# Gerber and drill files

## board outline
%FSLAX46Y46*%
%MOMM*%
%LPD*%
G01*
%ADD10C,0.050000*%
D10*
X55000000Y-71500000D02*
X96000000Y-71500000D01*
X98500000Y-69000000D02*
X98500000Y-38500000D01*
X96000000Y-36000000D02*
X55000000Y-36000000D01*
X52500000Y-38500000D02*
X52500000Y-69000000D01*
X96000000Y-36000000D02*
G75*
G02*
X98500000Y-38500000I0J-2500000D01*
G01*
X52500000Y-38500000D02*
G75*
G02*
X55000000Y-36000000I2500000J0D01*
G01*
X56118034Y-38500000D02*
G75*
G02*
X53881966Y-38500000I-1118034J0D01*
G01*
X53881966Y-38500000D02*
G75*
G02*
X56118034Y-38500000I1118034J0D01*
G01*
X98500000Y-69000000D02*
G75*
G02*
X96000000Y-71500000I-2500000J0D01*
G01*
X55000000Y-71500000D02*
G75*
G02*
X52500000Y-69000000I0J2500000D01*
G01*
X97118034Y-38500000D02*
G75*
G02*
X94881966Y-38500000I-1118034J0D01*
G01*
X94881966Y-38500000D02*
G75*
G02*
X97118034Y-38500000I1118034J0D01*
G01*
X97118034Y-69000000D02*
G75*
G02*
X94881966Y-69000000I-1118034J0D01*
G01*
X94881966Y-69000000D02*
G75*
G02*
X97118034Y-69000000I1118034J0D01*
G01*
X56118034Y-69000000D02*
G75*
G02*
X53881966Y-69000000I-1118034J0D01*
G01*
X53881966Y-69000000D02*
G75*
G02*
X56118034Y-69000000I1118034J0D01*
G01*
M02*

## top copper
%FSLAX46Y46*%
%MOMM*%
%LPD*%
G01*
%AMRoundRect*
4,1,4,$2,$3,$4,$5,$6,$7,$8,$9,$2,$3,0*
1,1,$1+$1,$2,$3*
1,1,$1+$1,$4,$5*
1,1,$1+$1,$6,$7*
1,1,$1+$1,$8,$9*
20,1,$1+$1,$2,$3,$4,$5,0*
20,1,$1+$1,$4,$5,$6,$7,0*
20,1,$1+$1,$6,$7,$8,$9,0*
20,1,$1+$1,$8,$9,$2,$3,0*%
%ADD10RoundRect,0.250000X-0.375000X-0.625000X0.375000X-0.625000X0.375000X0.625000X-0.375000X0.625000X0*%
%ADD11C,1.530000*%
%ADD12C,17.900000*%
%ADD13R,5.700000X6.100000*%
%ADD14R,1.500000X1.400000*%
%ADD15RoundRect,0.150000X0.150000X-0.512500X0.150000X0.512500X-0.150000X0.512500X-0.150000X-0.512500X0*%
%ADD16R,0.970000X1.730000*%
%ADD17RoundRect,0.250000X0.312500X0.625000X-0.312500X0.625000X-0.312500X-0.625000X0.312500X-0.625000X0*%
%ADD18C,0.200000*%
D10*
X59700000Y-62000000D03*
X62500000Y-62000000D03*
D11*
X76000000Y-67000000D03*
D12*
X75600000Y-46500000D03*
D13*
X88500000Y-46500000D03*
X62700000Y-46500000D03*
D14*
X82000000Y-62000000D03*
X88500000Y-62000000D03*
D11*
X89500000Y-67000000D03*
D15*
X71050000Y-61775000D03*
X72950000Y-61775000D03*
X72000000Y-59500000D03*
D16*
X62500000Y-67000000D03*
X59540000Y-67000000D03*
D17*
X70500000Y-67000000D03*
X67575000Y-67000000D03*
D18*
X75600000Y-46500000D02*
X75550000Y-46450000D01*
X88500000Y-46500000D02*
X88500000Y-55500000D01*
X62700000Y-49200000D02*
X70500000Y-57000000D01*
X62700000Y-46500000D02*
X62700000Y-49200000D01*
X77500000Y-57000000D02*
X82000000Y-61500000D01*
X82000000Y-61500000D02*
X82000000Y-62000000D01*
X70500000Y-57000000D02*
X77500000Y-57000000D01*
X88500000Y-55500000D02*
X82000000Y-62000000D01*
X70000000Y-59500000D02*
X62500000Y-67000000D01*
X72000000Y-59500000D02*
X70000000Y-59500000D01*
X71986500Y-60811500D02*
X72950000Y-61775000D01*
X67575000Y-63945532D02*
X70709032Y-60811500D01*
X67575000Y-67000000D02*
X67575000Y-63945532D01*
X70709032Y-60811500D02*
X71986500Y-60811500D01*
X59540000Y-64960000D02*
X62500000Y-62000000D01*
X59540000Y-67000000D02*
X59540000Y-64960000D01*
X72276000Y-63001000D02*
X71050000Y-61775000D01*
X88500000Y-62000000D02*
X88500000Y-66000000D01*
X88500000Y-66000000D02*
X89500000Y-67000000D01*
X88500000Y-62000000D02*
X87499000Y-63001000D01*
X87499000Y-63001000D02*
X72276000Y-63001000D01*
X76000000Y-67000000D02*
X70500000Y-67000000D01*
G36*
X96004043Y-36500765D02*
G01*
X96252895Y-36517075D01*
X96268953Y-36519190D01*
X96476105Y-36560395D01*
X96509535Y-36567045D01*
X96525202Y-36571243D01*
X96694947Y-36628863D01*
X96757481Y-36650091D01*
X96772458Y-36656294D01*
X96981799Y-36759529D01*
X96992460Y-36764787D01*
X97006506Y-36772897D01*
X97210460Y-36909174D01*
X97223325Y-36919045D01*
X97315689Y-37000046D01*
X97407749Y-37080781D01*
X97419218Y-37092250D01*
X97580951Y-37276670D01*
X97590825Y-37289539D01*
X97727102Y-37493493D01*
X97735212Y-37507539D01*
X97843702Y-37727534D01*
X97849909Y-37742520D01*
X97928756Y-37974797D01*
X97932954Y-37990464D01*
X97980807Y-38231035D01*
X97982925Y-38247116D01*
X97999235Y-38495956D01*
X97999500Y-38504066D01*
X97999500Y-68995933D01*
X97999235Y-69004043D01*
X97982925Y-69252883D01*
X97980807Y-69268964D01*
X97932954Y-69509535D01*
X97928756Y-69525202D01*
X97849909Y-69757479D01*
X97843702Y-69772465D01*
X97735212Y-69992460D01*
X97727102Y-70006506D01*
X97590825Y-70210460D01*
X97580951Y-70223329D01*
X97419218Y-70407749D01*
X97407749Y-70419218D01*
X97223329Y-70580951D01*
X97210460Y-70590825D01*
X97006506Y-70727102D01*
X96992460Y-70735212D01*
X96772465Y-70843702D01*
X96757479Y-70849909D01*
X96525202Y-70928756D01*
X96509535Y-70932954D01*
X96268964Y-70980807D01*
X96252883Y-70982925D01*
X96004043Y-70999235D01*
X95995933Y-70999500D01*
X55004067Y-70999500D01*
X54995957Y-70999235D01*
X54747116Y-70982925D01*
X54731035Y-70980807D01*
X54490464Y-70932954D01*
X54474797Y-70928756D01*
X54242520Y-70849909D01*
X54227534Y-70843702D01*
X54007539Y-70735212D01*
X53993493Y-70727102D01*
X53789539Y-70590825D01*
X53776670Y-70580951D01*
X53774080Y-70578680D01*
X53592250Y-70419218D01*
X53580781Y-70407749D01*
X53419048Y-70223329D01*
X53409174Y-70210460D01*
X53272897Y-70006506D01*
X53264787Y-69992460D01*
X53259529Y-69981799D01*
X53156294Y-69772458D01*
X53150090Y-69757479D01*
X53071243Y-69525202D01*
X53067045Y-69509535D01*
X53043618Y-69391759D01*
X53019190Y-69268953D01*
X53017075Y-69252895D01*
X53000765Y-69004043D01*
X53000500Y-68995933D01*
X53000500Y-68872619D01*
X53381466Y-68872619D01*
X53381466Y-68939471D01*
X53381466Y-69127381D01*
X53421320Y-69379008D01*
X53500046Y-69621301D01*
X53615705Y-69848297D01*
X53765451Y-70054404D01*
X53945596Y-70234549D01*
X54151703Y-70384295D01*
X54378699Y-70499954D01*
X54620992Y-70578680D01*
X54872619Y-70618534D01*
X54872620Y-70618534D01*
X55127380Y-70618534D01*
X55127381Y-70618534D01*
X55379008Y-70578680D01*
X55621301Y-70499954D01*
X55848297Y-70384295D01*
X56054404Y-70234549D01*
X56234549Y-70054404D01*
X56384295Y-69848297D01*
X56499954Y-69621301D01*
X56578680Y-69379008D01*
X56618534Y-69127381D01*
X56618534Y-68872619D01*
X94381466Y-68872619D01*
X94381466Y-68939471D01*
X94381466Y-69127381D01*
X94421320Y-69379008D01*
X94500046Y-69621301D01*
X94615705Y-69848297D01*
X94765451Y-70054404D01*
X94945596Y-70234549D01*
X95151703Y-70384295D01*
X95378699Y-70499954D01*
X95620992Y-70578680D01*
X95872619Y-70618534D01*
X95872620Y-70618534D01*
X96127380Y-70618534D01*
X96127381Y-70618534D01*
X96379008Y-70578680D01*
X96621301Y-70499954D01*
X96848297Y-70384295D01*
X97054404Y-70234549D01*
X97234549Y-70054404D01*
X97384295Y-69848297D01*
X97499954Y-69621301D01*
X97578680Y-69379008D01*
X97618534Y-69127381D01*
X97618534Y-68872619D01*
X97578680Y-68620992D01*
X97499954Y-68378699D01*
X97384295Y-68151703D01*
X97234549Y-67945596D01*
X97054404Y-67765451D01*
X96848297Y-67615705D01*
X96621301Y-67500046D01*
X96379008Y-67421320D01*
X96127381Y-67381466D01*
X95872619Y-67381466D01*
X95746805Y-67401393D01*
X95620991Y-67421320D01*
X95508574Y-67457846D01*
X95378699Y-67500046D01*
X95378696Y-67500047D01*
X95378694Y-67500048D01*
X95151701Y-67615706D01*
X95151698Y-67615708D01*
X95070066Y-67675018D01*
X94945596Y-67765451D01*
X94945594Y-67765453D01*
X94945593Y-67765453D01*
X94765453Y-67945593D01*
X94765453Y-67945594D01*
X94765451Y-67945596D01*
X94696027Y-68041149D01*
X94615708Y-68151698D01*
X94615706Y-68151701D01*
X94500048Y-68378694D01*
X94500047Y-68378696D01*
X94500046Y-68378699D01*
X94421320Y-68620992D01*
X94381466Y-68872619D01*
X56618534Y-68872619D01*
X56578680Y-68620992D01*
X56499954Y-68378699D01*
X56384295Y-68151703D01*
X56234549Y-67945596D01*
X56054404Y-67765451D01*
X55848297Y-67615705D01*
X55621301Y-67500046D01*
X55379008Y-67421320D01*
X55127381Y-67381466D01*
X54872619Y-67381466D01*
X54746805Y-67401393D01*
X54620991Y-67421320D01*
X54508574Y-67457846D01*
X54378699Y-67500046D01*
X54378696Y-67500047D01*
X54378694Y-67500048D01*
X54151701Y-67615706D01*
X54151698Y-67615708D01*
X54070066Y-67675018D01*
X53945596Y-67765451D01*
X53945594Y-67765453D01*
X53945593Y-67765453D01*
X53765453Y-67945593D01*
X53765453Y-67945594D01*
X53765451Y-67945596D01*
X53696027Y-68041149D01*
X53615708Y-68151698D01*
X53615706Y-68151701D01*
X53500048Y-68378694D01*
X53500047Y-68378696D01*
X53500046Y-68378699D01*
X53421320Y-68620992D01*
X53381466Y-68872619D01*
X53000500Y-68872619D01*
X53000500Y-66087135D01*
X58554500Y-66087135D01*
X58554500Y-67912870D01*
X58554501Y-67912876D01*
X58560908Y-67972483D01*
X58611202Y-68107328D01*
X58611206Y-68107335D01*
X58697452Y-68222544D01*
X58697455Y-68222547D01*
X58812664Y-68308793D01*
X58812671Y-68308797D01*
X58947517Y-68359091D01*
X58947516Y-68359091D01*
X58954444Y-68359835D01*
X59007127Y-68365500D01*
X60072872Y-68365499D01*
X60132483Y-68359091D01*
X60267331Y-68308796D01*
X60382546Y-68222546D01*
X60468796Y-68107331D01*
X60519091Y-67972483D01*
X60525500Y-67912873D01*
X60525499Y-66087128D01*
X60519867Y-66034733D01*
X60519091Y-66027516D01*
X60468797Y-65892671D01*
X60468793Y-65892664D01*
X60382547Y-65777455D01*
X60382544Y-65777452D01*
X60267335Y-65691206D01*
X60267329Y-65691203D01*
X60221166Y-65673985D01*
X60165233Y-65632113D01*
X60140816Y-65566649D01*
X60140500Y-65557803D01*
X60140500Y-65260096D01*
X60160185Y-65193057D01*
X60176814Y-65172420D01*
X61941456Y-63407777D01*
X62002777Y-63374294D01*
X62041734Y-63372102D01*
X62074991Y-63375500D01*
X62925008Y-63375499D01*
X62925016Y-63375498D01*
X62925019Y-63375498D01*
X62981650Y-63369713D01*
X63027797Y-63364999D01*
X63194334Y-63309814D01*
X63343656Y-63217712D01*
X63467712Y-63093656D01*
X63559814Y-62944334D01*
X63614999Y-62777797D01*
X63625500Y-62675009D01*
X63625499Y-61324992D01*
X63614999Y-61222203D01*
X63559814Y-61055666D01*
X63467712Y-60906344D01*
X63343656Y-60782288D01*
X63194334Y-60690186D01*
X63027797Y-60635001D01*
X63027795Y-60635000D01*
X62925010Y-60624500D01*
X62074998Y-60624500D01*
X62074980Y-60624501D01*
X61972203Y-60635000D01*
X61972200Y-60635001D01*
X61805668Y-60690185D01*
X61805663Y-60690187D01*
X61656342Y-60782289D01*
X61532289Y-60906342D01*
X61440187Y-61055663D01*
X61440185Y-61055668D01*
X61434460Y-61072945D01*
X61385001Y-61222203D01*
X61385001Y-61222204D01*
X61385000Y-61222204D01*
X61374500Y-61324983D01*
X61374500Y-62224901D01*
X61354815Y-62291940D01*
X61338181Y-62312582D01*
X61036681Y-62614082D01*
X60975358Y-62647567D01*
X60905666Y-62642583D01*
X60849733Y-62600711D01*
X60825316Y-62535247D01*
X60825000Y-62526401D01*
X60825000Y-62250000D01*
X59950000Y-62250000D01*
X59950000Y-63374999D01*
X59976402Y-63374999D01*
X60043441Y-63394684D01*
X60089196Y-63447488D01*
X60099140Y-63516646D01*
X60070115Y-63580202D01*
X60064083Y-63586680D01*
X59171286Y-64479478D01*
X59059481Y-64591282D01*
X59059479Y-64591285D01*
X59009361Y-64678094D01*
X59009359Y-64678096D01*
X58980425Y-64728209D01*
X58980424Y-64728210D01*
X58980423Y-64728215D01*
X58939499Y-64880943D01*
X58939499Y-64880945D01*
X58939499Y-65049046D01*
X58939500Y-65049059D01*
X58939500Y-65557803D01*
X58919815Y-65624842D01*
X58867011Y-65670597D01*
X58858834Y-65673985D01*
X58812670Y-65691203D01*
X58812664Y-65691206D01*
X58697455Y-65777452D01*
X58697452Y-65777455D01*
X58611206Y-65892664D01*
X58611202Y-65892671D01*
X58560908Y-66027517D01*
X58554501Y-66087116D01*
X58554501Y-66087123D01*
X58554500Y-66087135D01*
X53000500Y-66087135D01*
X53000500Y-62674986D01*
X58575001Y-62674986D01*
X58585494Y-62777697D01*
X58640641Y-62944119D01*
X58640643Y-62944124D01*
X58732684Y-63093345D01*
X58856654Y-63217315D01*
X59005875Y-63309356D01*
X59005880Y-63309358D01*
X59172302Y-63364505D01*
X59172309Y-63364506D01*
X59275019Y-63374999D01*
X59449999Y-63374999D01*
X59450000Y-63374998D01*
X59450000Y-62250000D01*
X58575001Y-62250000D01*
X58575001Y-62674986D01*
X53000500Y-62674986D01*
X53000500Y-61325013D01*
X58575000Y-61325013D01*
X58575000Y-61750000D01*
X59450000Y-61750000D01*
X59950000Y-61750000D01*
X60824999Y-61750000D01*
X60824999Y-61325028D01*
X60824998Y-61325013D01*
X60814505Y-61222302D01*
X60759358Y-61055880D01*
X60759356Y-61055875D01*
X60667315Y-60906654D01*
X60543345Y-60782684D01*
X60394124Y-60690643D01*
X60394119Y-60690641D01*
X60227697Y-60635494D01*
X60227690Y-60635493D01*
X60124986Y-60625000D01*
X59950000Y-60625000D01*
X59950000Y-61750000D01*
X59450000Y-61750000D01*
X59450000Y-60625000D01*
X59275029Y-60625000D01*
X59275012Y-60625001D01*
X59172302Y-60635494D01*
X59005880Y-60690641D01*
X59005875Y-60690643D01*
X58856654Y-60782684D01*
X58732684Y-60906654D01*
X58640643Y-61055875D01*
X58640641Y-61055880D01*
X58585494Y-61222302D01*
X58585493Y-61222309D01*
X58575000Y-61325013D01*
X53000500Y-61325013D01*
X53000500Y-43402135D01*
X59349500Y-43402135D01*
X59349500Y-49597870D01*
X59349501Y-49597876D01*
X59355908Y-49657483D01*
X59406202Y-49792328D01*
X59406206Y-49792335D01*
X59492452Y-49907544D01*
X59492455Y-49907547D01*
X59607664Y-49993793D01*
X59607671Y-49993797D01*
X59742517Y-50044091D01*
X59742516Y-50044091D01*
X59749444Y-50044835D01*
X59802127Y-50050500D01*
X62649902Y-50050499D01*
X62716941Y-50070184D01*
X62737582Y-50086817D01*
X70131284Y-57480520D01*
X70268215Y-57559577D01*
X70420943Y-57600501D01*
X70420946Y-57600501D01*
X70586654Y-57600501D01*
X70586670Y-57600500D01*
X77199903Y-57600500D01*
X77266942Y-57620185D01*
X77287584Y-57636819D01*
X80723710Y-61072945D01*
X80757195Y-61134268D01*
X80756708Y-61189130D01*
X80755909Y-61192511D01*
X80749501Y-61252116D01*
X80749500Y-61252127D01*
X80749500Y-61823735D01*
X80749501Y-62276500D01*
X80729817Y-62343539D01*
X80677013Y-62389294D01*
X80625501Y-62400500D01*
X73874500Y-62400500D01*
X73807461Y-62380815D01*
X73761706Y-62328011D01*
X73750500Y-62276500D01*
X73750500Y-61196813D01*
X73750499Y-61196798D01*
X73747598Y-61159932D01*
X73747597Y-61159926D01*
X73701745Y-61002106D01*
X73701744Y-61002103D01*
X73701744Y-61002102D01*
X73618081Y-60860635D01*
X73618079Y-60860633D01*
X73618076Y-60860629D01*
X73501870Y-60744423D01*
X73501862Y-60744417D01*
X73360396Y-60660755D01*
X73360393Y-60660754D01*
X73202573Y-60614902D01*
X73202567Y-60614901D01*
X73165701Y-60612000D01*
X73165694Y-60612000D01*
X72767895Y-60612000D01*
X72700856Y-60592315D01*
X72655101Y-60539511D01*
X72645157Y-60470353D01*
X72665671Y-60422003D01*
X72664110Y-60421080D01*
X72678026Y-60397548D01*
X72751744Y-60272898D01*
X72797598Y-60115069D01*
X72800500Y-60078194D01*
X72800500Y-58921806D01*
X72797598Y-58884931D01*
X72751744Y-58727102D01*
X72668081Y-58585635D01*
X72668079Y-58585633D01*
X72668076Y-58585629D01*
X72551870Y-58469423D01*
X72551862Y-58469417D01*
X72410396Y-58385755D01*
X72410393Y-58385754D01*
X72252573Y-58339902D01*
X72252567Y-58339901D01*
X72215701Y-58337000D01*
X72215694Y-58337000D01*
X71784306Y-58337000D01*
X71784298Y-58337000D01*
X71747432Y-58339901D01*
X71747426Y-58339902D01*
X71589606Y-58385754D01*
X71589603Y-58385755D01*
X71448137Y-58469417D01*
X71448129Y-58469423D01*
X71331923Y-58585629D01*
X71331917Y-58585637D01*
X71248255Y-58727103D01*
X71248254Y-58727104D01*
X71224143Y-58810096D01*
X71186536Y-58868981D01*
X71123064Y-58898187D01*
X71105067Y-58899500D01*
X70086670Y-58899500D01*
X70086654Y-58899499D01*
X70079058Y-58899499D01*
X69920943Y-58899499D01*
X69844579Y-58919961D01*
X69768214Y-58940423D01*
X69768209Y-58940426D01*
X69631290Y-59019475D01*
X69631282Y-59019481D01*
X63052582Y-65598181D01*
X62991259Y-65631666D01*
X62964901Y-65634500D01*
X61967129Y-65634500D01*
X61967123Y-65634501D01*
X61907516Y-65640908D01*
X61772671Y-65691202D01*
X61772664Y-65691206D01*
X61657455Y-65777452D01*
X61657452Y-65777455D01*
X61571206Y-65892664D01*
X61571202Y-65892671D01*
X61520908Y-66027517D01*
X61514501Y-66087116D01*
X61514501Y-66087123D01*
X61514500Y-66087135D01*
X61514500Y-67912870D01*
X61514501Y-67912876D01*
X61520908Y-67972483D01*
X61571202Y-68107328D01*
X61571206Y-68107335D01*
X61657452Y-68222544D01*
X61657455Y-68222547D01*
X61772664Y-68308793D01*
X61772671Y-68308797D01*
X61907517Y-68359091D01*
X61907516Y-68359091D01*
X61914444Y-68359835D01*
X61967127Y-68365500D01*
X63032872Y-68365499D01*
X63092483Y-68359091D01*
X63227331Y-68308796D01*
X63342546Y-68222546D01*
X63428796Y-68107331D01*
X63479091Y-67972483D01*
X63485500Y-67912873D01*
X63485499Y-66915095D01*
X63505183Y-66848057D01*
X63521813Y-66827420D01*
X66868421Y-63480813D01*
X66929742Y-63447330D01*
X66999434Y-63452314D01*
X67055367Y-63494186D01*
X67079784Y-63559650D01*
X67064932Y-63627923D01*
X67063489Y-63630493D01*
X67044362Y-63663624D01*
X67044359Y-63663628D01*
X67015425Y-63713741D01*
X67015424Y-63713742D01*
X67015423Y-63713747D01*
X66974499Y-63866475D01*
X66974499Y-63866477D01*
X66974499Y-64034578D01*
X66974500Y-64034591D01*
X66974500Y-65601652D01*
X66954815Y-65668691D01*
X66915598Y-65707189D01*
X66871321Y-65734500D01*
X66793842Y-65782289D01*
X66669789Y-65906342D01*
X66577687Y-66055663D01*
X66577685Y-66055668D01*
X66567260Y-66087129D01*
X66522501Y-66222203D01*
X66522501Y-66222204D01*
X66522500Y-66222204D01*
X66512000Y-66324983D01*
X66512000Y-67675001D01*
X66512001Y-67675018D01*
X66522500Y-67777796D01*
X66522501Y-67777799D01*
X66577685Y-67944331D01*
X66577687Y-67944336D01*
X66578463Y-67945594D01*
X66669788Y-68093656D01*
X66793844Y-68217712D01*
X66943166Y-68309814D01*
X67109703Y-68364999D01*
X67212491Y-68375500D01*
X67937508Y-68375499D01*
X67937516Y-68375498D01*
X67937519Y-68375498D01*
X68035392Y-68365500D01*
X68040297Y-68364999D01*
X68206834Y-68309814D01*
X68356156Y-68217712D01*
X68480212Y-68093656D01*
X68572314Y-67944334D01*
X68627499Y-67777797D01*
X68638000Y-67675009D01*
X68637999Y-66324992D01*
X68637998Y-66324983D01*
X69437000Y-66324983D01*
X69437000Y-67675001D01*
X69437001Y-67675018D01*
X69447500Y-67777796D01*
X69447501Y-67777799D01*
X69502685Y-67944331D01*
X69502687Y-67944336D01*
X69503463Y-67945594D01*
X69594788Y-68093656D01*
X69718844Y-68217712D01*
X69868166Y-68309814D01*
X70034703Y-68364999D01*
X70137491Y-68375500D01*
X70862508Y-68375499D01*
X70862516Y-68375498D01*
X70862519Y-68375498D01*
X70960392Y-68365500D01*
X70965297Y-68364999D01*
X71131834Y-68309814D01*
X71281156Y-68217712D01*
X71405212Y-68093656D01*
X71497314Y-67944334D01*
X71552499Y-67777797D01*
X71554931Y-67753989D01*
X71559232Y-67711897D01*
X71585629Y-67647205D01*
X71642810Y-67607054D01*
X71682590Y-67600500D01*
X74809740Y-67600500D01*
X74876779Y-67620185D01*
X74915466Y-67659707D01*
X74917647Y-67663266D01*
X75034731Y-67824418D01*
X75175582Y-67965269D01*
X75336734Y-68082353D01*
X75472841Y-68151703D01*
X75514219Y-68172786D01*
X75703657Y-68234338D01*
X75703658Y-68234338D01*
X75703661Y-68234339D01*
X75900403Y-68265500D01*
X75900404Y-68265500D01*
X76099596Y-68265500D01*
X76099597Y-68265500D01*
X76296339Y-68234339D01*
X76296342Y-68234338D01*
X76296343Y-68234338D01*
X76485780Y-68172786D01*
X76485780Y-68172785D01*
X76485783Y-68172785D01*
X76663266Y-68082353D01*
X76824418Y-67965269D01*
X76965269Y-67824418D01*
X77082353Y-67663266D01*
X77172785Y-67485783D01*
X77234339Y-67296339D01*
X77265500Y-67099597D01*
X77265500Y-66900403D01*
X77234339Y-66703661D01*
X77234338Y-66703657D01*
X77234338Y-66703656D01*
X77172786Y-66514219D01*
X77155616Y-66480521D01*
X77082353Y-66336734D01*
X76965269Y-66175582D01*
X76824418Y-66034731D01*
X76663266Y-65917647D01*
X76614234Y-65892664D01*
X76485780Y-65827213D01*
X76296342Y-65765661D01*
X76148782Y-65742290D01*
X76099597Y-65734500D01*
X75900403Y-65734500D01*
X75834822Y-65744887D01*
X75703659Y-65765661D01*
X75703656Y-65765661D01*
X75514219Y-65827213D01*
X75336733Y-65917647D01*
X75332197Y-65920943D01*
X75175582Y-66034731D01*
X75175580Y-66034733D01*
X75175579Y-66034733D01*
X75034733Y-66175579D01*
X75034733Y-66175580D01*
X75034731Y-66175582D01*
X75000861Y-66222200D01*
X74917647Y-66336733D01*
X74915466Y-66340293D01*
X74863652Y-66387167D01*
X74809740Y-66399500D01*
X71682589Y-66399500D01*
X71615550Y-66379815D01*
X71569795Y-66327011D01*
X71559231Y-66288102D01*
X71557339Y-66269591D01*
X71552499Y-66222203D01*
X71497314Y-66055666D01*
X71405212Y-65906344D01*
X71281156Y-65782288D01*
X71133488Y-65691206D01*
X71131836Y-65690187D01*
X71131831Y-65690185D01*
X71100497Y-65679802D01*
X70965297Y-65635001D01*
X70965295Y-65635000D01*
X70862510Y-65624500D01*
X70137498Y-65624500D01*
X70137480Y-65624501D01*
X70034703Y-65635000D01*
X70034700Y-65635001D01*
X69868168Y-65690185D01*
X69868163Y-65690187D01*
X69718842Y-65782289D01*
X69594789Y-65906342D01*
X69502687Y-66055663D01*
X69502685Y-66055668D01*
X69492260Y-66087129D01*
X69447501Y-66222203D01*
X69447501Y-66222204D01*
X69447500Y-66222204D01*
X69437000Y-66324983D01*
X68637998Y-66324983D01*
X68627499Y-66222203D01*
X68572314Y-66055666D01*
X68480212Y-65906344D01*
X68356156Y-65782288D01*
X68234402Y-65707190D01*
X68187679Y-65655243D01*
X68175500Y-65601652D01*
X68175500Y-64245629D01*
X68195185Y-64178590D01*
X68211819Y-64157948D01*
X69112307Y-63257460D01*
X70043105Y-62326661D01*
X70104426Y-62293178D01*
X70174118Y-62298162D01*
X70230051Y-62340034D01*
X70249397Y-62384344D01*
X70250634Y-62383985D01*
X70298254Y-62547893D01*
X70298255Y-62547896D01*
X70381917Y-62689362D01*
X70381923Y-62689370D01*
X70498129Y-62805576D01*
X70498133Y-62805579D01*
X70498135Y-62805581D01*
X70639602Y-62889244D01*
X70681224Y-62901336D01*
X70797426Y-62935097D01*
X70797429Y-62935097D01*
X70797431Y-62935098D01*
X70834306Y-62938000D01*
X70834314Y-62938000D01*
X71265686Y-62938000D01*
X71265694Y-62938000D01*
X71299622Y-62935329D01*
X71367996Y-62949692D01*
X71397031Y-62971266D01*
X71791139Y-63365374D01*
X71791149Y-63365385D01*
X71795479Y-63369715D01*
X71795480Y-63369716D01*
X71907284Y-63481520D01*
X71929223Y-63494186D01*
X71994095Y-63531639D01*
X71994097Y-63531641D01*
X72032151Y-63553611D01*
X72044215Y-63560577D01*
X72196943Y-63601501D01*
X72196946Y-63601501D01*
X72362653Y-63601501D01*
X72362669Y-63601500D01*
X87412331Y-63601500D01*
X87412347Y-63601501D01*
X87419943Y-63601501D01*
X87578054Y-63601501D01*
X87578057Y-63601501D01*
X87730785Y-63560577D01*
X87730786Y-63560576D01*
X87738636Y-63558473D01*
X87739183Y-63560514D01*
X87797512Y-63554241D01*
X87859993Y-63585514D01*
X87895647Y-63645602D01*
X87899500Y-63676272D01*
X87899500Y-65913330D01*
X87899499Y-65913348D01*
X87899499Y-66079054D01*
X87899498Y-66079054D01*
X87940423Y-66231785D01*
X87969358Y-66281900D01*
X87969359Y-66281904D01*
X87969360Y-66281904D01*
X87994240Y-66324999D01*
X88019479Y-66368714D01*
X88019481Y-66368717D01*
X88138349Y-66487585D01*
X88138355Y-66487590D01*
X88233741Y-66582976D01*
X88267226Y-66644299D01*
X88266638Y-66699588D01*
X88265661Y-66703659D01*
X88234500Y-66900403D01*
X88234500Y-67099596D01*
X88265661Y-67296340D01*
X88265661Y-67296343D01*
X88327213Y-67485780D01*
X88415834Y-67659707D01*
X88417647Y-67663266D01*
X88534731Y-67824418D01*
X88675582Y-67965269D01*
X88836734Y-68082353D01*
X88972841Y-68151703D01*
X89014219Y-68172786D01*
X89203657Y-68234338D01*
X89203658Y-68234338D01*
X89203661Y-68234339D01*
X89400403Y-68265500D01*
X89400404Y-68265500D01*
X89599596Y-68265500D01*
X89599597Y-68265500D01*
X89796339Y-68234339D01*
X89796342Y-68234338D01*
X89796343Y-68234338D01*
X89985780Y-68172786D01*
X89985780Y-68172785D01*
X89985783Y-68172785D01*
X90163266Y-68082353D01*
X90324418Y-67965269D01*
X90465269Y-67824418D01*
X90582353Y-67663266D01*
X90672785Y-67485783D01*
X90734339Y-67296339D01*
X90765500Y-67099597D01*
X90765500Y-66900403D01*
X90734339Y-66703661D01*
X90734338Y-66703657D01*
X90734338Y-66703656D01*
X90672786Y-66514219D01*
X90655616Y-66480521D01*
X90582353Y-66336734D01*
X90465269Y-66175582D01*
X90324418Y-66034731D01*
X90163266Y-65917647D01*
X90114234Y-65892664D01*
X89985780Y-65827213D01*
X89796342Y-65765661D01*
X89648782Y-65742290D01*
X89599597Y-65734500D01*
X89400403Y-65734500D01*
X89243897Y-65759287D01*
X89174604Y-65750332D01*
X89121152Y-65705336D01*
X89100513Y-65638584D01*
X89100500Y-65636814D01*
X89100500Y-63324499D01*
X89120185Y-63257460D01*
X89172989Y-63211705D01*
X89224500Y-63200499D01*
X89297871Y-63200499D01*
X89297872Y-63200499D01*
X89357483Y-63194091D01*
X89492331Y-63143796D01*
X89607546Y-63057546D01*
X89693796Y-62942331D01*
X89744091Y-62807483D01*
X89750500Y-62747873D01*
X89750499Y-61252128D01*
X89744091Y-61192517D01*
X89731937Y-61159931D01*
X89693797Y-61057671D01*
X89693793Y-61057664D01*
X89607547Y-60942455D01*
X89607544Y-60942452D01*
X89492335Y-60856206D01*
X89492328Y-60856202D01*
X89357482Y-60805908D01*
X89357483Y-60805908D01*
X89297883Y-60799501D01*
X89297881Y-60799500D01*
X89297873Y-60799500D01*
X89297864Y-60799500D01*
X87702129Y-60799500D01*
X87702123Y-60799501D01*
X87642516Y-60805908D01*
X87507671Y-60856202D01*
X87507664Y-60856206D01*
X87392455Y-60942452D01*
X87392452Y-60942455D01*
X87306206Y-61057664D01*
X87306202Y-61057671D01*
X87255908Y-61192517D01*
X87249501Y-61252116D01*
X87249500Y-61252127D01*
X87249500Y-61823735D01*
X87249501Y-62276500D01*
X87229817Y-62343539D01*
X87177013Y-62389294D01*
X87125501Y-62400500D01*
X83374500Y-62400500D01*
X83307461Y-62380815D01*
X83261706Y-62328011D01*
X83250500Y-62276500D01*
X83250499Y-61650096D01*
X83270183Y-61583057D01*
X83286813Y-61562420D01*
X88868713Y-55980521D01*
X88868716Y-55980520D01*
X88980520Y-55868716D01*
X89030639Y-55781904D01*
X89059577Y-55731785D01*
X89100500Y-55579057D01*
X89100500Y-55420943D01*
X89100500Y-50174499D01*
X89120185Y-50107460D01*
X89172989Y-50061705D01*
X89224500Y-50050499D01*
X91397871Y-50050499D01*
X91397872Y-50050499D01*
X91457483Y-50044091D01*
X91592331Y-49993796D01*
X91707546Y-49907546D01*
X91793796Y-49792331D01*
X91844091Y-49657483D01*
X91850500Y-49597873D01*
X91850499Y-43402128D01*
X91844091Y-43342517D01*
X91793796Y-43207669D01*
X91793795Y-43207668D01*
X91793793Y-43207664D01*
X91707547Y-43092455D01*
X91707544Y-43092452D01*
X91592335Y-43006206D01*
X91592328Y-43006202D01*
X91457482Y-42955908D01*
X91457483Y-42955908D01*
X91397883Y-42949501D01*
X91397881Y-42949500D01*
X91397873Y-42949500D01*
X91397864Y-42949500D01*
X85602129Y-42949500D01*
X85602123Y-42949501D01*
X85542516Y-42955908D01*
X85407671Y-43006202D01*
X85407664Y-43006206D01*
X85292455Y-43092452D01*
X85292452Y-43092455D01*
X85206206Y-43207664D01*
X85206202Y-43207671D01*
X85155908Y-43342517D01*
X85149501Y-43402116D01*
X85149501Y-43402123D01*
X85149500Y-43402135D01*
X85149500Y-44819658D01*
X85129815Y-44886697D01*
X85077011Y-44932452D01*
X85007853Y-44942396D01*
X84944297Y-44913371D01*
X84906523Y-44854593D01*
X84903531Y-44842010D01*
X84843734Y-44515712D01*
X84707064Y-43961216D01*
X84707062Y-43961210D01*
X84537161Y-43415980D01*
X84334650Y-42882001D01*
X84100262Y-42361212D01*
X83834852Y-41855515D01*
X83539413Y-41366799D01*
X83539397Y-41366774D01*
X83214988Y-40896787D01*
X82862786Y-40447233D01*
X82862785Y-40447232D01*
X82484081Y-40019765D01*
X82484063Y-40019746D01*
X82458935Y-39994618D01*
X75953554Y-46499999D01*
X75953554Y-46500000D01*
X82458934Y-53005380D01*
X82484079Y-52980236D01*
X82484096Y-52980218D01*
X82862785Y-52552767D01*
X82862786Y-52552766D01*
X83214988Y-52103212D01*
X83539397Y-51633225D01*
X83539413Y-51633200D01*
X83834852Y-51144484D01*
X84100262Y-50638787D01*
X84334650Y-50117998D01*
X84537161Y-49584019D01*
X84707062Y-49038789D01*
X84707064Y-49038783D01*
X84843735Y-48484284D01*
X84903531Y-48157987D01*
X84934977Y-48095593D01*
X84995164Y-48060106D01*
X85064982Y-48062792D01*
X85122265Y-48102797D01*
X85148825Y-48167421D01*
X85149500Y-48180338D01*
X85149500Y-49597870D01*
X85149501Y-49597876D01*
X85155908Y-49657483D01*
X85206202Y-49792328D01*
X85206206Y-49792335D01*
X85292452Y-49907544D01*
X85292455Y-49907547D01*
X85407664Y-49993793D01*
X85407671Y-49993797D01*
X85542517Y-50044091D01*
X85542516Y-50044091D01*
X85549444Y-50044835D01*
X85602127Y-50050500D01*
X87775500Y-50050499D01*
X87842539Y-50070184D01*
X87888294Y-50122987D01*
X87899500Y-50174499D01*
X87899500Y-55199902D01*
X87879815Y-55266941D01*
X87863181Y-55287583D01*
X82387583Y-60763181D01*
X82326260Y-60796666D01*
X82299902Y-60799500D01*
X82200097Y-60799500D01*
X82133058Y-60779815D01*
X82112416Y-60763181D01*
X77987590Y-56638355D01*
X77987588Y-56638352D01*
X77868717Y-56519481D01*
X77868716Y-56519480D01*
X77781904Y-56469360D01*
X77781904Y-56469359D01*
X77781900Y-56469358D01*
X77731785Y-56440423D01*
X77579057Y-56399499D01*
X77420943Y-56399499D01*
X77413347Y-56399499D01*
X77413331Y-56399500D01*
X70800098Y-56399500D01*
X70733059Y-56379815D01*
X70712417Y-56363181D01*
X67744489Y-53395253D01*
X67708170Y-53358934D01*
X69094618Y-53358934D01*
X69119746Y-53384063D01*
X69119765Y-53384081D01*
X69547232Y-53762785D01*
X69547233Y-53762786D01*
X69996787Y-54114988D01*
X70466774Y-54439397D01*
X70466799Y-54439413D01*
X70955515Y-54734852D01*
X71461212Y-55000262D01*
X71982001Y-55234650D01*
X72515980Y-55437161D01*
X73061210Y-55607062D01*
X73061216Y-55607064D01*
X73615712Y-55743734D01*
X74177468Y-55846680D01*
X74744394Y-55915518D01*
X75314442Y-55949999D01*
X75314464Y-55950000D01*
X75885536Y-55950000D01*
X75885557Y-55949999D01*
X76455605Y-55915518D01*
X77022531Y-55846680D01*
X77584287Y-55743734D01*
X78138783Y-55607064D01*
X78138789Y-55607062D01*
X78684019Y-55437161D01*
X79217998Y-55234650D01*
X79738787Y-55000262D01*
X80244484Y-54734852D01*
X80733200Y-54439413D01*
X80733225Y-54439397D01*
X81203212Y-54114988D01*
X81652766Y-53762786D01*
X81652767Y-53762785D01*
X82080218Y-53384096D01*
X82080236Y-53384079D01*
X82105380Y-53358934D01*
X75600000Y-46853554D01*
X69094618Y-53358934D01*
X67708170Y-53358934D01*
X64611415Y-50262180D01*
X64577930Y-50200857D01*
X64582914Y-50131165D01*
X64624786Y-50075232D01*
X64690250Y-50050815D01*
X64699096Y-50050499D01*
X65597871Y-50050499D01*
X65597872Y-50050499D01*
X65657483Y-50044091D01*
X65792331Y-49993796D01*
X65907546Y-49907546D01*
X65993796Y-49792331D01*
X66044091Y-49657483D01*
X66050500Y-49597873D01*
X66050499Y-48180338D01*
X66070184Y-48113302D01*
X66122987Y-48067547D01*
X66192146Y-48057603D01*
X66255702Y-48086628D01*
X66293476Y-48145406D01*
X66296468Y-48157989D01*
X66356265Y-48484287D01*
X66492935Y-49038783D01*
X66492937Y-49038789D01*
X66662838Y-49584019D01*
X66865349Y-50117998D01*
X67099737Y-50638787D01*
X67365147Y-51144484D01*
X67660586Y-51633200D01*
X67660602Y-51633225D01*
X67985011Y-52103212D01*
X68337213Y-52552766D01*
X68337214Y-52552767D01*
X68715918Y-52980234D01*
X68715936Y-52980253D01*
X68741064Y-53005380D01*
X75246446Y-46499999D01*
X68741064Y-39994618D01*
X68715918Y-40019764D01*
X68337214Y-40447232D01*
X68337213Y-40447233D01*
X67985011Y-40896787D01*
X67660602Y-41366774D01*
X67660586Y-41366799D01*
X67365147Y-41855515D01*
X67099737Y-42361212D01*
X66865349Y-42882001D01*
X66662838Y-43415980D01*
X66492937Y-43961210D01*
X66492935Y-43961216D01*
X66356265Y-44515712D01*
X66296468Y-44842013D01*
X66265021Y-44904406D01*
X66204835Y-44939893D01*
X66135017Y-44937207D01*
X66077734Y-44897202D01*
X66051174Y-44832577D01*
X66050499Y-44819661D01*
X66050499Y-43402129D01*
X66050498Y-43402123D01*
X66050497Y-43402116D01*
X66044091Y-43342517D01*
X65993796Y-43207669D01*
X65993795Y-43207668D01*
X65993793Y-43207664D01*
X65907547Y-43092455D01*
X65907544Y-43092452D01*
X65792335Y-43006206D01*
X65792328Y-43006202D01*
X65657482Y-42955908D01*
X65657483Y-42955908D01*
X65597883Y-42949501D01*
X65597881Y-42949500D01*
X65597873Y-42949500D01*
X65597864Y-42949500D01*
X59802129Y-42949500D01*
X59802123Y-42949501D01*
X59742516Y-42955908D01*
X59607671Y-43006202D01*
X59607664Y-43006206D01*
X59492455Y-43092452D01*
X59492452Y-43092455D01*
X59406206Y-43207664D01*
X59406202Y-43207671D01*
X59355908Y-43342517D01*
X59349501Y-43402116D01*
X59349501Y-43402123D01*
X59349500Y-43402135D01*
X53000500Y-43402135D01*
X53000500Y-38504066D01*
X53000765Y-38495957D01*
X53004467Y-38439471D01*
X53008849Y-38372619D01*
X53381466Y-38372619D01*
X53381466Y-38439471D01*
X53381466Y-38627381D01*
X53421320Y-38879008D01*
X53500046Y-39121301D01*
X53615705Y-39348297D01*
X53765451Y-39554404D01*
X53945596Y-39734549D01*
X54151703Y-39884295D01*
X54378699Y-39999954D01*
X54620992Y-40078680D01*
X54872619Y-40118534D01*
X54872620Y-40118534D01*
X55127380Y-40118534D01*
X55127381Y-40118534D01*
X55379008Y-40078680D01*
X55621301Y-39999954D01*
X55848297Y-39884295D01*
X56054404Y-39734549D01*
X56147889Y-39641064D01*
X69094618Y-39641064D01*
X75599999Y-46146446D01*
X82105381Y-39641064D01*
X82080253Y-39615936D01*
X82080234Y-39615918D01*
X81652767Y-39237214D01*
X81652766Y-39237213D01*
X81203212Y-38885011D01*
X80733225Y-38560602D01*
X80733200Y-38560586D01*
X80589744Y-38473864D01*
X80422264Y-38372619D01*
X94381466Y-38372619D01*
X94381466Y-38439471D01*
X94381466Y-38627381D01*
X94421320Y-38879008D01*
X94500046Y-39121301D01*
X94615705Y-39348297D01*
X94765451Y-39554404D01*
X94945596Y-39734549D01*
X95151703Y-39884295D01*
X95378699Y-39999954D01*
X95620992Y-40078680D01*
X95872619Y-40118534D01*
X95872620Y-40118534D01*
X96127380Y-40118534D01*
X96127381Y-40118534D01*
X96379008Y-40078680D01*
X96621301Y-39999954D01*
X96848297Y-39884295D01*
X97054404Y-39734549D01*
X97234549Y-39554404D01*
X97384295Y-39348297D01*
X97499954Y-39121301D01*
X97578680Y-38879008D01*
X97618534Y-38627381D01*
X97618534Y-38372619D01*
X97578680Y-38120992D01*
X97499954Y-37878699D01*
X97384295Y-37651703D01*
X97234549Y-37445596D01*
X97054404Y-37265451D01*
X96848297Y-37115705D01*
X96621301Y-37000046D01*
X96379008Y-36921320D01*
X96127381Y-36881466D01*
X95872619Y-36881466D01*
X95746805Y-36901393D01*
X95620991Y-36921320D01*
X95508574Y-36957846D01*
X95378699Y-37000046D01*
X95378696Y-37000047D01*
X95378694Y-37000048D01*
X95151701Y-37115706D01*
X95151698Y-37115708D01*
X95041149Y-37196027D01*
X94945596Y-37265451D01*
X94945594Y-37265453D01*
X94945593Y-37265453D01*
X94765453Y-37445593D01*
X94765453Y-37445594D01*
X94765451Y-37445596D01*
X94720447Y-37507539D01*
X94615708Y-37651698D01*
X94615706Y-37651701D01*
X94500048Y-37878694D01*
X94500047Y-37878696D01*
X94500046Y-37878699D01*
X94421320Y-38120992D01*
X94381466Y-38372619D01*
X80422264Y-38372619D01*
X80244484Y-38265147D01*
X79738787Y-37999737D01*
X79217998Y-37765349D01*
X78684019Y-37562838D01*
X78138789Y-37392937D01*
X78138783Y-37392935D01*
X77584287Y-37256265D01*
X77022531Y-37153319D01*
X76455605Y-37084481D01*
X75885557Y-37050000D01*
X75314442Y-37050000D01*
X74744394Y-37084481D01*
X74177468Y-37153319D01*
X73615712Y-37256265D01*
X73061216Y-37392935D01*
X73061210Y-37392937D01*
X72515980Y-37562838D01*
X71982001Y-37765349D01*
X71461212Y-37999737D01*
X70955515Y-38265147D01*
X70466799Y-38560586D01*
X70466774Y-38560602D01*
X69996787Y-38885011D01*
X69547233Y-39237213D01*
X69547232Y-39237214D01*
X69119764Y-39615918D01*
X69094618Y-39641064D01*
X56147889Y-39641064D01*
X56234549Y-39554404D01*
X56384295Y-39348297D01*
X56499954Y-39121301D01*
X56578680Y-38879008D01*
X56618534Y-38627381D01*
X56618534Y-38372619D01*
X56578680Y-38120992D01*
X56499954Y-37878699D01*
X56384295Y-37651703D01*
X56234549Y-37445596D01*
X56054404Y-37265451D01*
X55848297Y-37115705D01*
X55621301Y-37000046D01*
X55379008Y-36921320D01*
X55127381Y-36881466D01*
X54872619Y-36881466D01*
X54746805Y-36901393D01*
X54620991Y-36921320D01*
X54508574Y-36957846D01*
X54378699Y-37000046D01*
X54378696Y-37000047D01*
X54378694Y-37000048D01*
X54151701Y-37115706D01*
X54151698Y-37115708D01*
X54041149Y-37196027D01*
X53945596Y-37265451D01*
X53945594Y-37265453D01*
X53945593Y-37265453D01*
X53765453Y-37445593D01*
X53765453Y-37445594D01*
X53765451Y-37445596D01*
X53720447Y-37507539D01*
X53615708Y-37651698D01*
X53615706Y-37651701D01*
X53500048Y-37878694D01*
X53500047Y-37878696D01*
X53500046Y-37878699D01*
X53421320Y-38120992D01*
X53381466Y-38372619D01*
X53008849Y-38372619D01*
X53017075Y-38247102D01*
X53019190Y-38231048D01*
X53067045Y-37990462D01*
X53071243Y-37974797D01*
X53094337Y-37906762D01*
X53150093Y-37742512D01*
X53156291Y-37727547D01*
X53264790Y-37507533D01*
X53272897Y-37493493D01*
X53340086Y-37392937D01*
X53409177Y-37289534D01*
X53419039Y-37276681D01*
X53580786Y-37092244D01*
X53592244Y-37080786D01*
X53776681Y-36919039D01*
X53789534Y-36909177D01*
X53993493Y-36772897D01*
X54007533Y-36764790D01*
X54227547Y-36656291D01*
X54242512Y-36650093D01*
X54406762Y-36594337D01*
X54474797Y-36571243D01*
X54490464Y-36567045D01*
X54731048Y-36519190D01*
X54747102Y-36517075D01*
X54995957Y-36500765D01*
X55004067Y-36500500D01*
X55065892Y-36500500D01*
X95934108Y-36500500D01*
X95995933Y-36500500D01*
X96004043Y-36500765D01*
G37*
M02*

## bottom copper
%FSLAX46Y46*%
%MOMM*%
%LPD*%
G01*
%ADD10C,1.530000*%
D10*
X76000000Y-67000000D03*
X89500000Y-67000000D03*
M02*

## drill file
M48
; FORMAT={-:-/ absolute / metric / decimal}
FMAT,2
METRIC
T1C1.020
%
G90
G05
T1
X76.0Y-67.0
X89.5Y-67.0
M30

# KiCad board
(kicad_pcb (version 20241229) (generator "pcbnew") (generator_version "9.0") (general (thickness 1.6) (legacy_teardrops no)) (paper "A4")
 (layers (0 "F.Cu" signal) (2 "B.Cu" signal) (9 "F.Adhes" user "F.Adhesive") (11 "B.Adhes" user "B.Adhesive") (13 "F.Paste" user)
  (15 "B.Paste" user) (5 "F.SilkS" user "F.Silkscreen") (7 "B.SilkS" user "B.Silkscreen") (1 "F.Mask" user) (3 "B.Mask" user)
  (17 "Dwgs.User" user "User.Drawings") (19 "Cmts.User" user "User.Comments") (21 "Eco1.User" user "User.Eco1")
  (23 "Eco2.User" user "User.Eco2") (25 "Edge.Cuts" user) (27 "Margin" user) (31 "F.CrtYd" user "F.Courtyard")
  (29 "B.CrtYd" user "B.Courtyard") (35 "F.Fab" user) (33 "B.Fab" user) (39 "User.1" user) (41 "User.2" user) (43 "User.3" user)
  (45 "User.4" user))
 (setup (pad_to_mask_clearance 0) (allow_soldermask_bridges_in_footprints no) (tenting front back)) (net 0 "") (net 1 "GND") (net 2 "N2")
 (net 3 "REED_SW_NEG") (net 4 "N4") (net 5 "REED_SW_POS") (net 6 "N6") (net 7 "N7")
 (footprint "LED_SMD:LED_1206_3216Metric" (layer "F.Cu") (at 61.1 62)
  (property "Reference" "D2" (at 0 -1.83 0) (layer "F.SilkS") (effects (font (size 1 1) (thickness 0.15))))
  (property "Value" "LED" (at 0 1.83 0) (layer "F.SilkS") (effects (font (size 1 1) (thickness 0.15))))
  (pad "1" smd roundrect (at -1.4 0) (size 1.25 1.75) (layers "F.Cu" "F.Mask" "F.Paste") (roundrect_rratio 0.2) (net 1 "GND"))
  (pad "2" smd roundrect (at 1.4 0) (size 1.25 1.75) (layers "F.Cu" "F.Mask" "F.Paste") (roundrect_rratio 0.2) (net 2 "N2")))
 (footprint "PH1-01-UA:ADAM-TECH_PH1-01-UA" (layer "F.Cu") (at 76 67)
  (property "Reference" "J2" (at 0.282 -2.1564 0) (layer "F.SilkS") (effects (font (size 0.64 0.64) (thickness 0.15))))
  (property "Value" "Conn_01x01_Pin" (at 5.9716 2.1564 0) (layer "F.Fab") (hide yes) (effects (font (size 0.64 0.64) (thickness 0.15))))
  (pad "1" thru_hole circle (at 0 0) (size 1.53 1.53) (drill 1.02) (layers "*.Cu" "*.Mask") (remove_unused_layers no) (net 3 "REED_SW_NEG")
   (solder_mask_margin 0.102)))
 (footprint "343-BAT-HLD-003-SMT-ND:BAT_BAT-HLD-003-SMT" (layer "F.Cu") (at 75.6 46.5 180)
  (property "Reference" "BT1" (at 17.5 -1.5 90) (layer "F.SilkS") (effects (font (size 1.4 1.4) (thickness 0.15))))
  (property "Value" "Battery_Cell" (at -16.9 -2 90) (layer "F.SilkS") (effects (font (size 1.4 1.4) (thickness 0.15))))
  (pad "N" smd circle (at 0 0 180) (size 17.9 17.9) (layers "F.Cu" "F.Mask") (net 1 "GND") (solder_mask_margin 0.102))
  (pad "P1" smd rect (at -12.9 0 180) (size 5.7 6.1) (layers "F.Cu" "F.Mask" "F.Paste") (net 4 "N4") (solder_mask_margin 0.102))
  (pad "P1" smd rect (at 12.9 0 180) (size 5.7 6.1) (layers "F.Cu" "F.Mask" "F.Paste") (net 4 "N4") (solder_mask_margin 0.102)))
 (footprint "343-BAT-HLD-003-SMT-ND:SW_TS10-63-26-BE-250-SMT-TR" (layer "F.Cu") (at 85.25 62)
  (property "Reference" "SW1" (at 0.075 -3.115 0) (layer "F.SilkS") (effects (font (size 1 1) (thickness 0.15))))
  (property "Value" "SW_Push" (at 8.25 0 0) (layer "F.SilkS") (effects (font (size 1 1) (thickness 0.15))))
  (pad "1" smd rect (at -3.25 0) (size 1.5 1.4) (layers "F.Cu" "F.Mask" "F.Paste") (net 4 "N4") (solder_mask_margin 0.102))
  (pad "2" smd rect (at 3.25 0) (size 1.5 1.4) (layers "F.Cu" "F.Mask" "F.Paste") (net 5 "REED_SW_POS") (solder_mask_margin 0.102)))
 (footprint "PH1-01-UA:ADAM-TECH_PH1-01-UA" (layer "F.Cu") (at 89.5 67)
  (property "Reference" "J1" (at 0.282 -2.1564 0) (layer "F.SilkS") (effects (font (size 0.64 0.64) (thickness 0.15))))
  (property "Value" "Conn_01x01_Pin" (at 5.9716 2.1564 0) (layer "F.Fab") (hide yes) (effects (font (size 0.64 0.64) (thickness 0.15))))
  (pad "1" thru_hole circle (at 0 0) (size 1.53 1.53) (drill 1.02) (layers "*.Cu" "*.Mask") (remove_unused_layers no) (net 5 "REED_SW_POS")
   (solder_mask_margin 0.102)))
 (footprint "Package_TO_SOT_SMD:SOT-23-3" (layer "F.Cu") (at 72 60.6375 90)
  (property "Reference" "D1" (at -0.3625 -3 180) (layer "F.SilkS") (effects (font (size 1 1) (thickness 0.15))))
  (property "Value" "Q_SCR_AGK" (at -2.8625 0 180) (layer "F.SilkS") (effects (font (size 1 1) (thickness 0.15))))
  (pad "1" smd roundrect (at -1.1375 -0.95 90) (size 1.325 0.6) (layers "F.Cu" "F.Mask" "F.Paste") (roundrect_rratio 0.25)
   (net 5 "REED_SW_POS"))
  (pad "2" smd roundrect (at -1.1375 0.95 90) (size 1.325 0.6) (layers "F.Cu" "F.Mask" "F.Paste") (roundrect_rratio 0.25) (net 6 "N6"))
  (pad "3" smd roundrect (at 1.1375 0 90) (size 1.325 0.6) (layers "F.Cu" "F.Mask" "F.Paste") (roundrect_rratio 0.25) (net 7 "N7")))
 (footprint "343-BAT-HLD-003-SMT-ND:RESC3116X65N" (layer "F.Cu") (at 61.02 67 180)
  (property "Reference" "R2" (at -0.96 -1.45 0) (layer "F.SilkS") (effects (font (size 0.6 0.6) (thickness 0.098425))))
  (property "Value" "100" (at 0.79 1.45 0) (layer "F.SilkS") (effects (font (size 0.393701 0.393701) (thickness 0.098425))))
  (pad "1" smd rect (at -1.48 0 180) (size 0.97 1.73) (layers "F.Cu" "F.Mask" "F.Paste") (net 7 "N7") (solder_mask_margin 0.102))
  (pad "2" smd rect (at 1.48 0 180) (size 0.97 1.73) (layers "F.Cu" "F.Mask" "F.Paste") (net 2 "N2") (solder_mask_margin 0.102)))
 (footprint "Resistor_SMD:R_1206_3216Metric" (layer "F.Cu") (at 69.0375 67 180)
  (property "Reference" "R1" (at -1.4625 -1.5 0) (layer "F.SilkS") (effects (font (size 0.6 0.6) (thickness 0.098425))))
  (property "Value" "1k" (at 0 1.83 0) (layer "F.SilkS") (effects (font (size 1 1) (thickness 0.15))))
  (pad "1" smd roundrect (at -1.4625 0 180) (size 1.125 1.75) (layers "F.Cu" "F.Mask" "F.Paste") (roundrect_rratio 0.222222)
   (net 3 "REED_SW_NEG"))
  (pad "2" smd roundrect (at 1.4625 0 180) (size 1.125 1.75) (layers "F.Cu" "F.Mask" "F.Paste") (roundrect_rratio 0.222222) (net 6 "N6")))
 (gr_line (start 55 71.5) (end 96 71.5) (stroke (width 0.05) (type default)) (layer "Edge.Cuts"))
 (gr_line (start 98.5 69) (end 98.5 38.5) (stroke (width 0.05) (type default)) (layer "Edge.Cuts"))
 (gr_line (start 96 36) (end 55 36) (stroke (width 0.05) (type default)) (layer "Edge.Cuts"))
 (gr_line (start 52.5 38.5) (end 52.5 69) (stroke (width 0.05) (type default)) (layer "Edge.Cuts"))
 (gr_arc (start 96 36) (mid 97.767767 36.732233) (end 98.5 38.5) (stroke (width 0.05) (type default)) (layer "Edge.Cuts"))
 (gr_arc (start 52.5 38.5) (mid 53.232233 36.732233) (end 55 36) (stroke (width 0.05) (type default)) (layer "Edge.Cuts"))
 (gr_circle (center 55 38.5) (end 56 39) (stroke (width 0.05) (type default)) (fill no) (layer "Edge.Cuts"))
 (gr_arc (start 98.5 69) (mid 97.767767 70.767767) (end 96 71.5) (stroke (width 0.05) (type default)) (layer "Edge.Cuts"))
 (gr_arc (start 55 71.5) (mid 53.232233 70.767767) (end 52.5 69) (stroke (width 0.05) (type default)) (layer "Edge.Cuts"))
 (gr_circle (center 96 38.5) (end 97 38) (stroke (width 0.05) (type default)) (fill no) (layer "Edge.Cuts"))
 (gr_circle (center 96 69) (end 97 69.5) (stroke (width 0.05) (type default)) (fill no) (layer "Edge.Cuts"))
 (gr_circle (center 55 69) (end 56 69.5) (stroke (width 0.05) (type default)) (fill no) (layer "Edge.Cuts"))
 (segment (start 75.6 46.5) (end 75.55 46.45) (width 0.2) (layer "F.Cu") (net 1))
 (segment (start 88.5 46.5) (end 88.5 55.5) (width 0.2) (layer "F.Cu") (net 4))
 (segment (start 62.7 49.2) (end 70.5 57) (width 0.2) (layer "F.Cu") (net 4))
 (segment (start 62.7 46.5) (end 62.7 49.2) (width 0.2) (layer "F.Cu") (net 4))
 (segment (start 77.5 57) (end 82 61.5) (width 0.2) (layer "F.Cu") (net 4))
 (segment (start 82 61.5) (end 82 62) (width 0.2) (layer "F.Cu") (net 4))
 (segment (start 70.5 57) (end 77.5 57) (width 0.2) (layer "F.Cu") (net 4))
 (segment (start 88.5 55.5) (end 82 62) (width 0.2) (layer "F.Cu") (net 4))
 (segment (start 70 59.5) (end 62.5 67) (width 0.2) (layer "F.Cu") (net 7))
 (segment (start 72 59.5) (end 70 59.5) (width 0.2) (layer "F.Cu") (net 7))
 (segment (start 71.9865 60.8115) (end 72.95 61.775) (width 0.2) (layer "F.Cu") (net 6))
 (segment (start 67.575 63.945532) (end 70.709032 60.8115) (width 0.2) (layer "F.Cu") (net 6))
 (segment (start 67.575 67) (end 67.575 63.945532) (width 0.2) (layer "F.Cu") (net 6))
 (segment (start 70.709032 60.8115) (end 71.9865 60.8115) (width 0.2) (layer "F.Cu") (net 6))
 (segment (start 59.54 64.96) (end 62.5 62) (width 0.2) (layer "F.Cu") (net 2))
 (segment (start 59.54 67) (end 59.54 64.96) (width 0.2) (layer "F.Cu") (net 2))
 (segment (start 72.276 63.001) (end 71.05 61.775) (width 0.2) (layer "F.Cu") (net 5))
 (segment (start 88.5 62) (end 88.5 66) (width 0.2) (layer "F.Cu") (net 5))
 (segment (start 88.5 66) (end 89.5 67) (width 0.2) (layer "F.Cu") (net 5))
 (segment (start 88.5 62) (end 87.499 63.001) (width 0.2) (layer "F.Cu") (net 5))
 (segment (start 87.499 63.001) (end 72.276 63.001) (width 0.2) (layer "F.Cu") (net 5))
 (segment (start 76 67) (end 70.5 67) (width 0.2) (layer "F.Cu") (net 3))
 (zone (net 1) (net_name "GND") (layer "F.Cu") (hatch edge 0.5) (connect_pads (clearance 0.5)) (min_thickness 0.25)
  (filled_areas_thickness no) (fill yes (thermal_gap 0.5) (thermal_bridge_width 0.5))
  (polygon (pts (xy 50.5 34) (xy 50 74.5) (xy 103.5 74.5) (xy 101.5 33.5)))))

